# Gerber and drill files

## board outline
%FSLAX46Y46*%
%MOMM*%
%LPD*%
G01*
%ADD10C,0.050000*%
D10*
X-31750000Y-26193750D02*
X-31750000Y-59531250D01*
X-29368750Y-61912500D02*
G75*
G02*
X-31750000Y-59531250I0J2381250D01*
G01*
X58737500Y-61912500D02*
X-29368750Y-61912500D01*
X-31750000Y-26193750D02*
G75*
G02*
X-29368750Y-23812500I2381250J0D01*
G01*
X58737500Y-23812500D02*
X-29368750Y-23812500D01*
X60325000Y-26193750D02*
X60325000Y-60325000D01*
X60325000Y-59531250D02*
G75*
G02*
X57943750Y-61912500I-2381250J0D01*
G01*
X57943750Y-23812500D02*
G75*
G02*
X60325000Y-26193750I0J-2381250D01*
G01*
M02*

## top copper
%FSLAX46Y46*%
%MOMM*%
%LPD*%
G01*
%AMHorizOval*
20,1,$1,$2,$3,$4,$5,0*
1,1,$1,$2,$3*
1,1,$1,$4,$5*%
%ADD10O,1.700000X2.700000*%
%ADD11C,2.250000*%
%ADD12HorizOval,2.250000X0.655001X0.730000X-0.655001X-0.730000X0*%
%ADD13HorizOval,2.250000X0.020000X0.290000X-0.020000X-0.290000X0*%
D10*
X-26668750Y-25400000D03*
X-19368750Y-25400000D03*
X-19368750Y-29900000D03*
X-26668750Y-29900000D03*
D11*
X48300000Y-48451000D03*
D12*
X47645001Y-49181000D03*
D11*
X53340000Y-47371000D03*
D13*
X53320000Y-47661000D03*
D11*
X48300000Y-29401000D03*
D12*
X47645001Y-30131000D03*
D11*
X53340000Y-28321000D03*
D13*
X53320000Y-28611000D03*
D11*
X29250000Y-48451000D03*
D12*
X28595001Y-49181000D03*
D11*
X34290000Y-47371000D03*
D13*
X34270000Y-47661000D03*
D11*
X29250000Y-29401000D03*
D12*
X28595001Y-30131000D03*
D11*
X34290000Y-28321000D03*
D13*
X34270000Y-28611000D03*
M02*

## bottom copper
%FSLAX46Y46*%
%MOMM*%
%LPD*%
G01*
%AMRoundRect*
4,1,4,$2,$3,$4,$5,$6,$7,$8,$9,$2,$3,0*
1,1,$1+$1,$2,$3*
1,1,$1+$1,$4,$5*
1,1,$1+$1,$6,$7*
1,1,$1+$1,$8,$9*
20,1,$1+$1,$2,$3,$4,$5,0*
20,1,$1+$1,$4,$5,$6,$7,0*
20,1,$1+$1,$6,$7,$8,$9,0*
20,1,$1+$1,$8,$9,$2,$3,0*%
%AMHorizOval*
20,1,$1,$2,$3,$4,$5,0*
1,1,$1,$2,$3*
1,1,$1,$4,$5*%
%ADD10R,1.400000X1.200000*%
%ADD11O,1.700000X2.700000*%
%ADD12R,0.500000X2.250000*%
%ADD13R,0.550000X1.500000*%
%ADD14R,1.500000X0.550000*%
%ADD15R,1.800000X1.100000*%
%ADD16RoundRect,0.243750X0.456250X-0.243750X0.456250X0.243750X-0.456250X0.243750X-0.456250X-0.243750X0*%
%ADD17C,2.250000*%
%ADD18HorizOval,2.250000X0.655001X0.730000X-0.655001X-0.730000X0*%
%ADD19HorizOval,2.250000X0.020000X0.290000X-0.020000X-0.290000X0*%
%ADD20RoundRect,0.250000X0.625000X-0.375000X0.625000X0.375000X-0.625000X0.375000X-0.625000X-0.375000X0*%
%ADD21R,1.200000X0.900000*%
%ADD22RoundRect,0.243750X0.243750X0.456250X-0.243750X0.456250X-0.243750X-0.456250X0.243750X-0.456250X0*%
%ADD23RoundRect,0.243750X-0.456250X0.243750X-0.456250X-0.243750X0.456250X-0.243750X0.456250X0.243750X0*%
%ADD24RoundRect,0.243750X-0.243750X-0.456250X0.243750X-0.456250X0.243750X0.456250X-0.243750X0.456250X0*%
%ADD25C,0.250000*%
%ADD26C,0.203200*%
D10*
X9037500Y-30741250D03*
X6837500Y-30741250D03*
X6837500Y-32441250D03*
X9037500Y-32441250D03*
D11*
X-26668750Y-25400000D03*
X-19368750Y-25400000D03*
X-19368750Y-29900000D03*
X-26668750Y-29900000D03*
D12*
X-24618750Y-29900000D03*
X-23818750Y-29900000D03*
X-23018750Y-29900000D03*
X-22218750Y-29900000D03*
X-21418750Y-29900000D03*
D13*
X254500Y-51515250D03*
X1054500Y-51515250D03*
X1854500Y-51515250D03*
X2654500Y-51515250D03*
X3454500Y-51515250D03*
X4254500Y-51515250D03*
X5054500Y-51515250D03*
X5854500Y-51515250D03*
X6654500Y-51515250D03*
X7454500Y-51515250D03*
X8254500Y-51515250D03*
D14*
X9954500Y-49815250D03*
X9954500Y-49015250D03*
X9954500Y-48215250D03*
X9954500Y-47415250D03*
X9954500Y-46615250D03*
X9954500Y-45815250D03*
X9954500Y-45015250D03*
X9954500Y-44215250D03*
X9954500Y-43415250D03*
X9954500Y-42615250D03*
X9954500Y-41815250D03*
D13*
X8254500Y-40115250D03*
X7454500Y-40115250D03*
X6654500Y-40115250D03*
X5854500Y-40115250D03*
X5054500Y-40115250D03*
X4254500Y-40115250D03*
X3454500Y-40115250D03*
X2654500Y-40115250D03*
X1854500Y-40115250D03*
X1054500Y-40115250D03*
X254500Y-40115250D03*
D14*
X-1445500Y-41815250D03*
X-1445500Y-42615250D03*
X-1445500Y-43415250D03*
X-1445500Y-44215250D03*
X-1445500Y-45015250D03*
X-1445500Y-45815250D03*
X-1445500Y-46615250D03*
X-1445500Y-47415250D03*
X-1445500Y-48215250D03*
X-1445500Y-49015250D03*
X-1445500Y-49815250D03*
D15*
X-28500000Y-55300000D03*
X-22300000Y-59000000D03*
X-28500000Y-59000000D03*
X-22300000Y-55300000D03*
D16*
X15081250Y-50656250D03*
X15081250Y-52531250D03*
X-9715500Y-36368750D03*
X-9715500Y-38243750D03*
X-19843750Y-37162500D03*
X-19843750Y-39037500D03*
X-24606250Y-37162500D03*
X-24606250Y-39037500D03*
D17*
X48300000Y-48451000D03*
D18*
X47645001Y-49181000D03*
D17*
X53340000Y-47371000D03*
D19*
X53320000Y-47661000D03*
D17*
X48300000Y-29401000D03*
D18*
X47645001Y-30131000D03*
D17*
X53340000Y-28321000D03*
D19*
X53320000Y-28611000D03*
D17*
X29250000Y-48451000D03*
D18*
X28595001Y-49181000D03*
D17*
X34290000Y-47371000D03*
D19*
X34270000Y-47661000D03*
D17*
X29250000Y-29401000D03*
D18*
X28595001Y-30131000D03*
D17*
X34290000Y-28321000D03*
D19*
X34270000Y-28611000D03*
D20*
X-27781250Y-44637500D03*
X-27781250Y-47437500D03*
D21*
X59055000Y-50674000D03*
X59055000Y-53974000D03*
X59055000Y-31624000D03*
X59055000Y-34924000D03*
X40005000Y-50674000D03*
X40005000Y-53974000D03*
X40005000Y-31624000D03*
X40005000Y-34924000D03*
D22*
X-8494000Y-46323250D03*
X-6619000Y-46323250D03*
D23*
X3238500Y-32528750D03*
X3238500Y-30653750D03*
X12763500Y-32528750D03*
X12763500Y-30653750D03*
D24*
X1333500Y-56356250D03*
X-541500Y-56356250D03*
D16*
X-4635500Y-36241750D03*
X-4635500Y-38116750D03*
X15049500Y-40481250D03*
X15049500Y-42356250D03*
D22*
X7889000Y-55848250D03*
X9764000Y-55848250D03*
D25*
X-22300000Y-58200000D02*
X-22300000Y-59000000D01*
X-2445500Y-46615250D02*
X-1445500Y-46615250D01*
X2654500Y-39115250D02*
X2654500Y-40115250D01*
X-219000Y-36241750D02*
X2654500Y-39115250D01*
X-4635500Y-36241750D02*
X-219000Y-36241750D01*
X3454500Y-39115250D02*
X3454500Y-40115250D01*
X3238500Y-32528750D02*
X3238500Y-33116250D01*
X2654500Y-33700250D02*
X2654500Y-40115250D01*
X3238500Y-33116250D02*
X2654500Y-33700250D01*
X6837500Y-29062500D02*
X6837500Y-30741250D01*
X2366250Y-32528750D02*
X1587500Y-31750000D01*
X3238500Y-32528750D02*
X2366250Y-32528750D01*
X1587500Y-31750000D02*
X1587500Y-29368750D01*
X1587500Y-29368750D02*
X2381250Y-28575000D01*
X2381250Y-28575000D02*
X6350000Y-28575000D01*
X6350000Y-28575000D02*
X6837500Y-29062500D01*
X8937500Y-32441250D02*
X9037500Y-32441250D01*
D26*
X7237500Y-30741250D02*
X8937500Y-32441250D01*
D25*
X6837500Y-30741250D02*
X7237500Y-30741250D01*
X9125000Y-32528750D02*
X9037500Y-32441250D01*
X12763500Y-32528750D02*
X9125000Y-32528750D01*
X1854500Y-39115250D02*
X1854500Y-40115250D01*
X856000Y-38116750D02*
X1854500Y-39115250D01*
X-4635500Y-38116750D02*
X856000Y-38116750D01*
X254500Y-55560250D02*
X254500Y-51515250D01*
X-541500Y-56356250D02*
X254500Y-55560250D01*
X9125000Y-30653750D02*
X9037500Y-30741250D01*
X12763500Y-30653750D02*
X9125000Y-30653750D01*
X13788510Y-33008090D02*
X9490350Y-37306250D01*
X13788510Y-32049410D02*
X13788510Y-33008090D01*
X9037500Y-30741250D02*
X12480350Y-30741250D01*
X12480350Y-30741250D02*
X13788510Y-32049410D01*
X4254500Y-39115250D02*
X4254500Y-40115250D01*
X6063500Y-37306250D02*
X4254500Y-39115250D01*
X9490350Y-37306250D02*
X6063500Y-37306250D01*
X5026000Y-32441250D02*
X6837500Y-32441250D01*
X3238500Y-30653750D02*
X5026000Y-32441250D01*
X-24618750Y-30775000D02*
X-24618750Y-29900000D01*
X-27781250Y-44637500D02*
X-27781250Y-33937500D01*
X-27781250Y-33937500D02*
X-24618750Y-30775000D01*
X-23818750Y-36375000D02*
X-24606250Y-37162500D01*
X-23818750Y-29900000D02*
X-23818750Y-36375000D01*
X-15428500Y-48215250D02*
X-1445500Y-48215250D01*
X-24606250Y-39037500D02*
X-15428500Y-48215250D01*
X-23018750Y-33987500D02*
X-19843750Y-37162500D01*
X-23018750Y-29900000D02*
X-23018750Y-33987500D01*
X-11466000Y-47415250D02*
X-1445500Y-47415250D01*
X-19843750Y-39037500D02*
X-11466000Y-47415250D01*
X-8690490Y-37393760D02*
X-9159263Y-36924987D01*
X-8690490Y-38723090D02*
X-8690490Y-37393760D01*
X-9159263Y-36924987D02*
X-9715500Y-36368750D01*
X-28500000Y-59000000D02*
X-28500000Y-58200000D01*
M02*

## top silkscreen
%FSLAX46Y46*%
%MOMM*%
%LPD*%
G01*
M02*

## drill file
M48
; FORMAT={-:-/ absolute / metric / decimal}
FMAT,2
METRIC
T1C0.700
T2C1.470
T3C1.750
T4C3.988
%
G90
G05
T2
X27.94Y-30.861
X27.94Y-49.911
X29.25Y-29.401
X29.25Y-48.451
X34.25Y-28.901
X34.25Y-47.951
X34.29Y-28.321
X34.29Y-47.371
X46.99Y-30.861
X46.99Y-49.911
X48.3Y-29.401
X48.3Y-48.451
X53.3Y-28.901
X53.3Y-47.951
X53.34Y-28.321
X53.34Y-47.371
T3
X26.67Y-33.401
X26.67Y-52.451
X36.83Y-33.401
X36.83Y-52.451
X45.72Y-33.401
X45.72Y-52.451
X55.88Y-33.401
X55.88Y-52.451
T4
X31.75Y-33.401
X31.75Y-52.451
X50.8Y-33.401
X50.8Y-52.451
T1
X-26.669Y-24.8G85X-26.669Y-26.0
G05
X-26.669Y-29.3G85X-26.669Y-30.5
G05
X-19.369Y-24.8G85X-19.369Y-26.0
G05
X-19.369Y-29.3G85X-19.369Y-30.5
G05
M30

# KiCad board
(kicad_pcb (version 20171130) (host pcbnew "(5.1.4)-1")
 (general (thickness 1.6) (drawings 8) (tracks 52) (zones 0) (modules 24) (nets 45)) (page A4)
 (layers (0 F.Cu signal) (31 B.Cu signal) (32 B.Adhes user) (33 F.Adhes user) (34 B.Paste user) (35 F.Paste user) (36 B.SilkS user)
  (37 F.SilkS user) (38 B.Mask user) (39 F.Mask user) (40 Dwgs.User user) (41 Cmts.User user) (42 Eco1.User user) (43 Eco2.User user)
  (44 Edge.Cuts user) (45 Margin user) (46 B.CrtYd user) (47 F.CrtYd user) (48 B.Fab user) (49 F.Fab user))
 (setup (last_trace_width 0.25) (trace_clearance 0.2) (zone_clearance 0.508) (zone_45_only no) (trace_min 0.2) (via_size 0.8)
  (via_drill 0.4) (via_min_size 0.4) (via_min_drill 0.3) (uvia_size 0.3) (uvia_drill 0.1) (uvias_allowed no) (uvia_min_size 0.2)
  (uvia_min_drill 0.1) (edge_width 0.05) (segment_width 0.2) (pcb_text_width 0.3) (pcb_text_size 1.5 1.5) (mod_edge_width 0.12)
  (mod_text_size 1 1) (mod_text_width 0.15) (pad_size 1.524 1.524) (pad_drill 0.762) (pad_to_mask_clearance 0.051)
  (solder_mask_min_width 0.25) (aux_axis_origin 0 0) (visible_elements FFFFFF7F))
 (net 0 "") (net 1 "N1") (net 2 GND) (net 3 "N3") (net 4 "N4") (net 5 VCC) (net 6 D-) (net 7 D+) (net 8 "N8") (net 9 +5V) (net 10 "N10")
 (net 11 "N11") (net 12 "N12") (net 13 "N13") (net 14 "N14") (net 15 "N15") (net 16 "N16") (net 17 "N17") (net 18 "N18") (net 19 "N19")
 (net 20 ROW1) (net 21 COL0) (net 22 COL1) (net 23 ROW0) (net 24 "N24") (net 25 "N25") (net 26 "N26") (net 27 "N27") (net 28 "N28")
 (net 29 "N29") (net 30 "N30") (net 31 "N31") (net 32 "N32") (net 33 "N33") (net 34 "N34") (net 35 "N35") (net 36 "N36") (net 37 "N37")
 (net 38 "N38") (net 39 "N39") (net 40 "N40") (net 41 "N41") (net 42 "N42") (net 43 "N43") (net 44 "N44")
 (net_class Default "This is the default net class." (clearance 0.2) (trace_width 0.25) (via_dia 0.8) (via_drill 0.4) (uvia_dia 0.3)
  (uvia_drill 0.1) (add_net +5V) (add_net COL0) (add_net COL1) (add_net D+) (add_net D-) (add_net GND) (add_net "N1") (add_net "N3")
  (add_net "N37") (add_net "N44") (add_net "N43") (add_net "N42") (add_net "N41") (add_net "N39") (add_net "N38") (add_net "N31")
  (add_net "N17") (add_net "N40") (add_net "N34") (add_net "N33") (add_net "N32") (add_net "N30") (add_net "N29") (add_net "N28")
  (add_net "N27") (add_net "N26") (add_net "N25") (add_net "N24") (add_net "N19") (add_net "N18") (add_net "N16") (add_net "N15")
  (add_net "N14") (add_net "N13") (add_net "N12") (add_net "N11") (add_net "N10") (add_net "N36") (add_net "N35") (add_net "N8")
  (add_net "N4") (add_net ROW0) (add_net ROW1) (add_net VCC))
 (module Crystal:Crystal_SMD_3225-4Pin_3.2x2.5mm (layer B.Cu) (at 7.9375 31.59125 180)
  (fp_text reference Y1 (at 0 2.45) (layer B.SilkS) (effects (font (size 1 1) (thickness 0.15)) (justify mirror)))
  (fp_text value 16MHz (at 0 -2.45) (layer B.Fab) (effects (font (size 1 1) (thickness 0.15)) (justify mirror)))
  (pad 4 smd rect (at -1.1 0.85 180) (size 1.4 1.2) (layers B.Cu B.Paste B.Mask) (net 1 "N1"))
  (pad 3 smd rect (at 1.1 0.85 180) (size 1.4 1.2) (layers B.Cu B.Paste B.Mask) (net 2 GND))
  (pad 2 smd rect (at 1.1 -0.85 180) (size 1.4 1.2) (layers B.Cu B.Paste B.Mask) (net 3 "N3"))
  (pad 1 smd rect (at -1.1 -0.85 180) (size 1.4 1.2) (layers B.Cu B.Paste B.Mask) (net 2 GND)))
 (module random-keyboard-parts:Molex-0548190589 (layer B.Cu) (at -23.01875 25.4 270)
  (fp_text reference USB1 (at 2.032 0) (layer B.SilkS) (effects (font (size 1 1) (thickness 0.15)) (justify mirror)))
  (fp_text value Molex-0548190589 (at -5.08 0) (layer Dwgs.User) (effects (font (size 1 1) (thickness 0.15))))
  (pad 6 thru_hole oval (at 0 3.65 270) (size 2.7 1.7) (drill oval 1.9 0.7) (layers *.Cu *.Mask) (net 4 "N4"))
  (pad 6 thru_hole oval (at 0 -3.65 270) (size 2.7 1.7) (drill oval 1.9 0.7) (layers *.Cu *.Mask) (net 4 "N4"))
  (pad 6 thru_hole oval (at 4.5 -3.65 270) (size 2.7 1.7) (drill oval 1.9 0.7) (layers *.Cu *.Mask) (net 4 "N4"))
  (pad 6 thru_hole oval (at 4.5 3.65 270) (size 2.7 1.7) (drill oval 1.9 0.7) (layers *.Cu *.Mask) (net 4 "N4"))
  (pad 5 smd rect (at 4.5 1.6 270) (size 2.25 0.5) (layers B.Cu B.Paste B.Mask) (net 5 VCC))
  (pad 4 smd rect (at 4.5 0.8 270) (size 2.25 0.5) (layers B.Cu B.Paste B.Mask) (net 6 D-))
  (pad 3 smd rect (at 4.5 0 270) (size 2.25 0.5) (layers B.Cu B.Paste B.Mask) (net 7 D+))
  (pad 2 smd rect (at 4.5 -0.8 270) (size 2.25 0.5) (layers B.Cu B.Paste B.Mask) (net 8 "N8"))
  (pad 1 smd rect (at 4.5 -1.6 270) (size 2.25 0.5) (layers B.Cu B.Paste B.Mask) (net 2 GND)))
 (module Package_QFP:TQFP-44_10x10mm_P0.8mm (layer B.Cu) (at 4.2545 45.81525)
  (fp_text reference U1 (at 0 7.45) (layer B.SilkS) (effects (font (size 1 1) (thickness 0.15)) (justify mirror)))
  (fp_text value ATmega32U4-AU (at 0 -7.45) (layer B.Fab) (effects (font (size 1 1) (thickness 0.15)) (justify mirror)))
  (pad 44 smd rect (at -4 5.7 270) (size 1.5 0.55) (layers B.Cu B.Paste B.Mask) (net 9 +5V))
  (pad 43 smd rect (at -3.2 5.7 270) (size 1.5 0.55) (layers B.Cu B.Paste B.Mask) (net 2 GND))
  (pad 42 smd rect (at -2.4 5.7 270) (size 1.5 0.55) (layers B.Cu B.Paste B.Mask) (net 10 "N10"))
  (pad 41 smd rect (at -1.6 5.7 270) (size 1.5 0.55) (layers B.Cu B.Paste B.Mask) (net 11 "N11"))
  (pad 40 smd rect (at -0.8 5.7 270) (size 1.5 0.55) (layers B.Cu B.Paste B.Mask) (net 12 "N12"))
  (pad 39 smd rect (at 0 5.7 270) (size 1.5 0.55) (layers B.Cu B.Paste B.Mask) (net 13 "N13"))
  (pad 38 smd rect (at 0.8 5.7 270) (size 1.5 0.55) (layers B.Cu B.Paste B.Mask) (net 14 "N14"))
  (pad 37 smd rect (at 1.6 5.7 270) (size 1.5 0.55) (layers B.Cu B.Paste B.Mask) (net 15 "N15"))
  (pad 36 smd rect (at 2.4 5.7 270) (size 1.5 0.55) (layers B.Cu B.Paste B.Mask) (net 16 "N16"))
  (pad 35 smd rect (at 3.2 5.7 270) (size 1.5 0.55) (layers B.Cu B.Paste B.Mask) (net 2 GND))
  (pad 34 smd rect (at 4 5.7 270) (size 1.5 0.55) (layers B.Cu B.Paste B.Mask) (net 9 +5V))
  (pad 33 smd rect (at 5.7 4) (size 1.5 0.55) (layers B.Cu B.Paste B.Mask) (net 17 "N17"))
  (pad 32 smd rect (at 5.7 3.2) (size 1.5 0.55) (layers B.Cu B.Paste B.Mask) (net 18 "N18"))
  (pad 31 smd rect (at 5.7 2.4) (size 1.5 0.55) (layers B.Cu B.Paste B.Mask) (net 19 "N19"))
  (pad 30 smd rect (at 5.7 1.6) (size 1.5 0.55) (layers B.Cu B.Paste B.Mask) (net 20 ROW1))
  (pad 29 smd rect (at 5.7 0.8) (size 1.5 0.55) (layers B.Cu B.Paste B.Mask) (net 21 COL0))
  (pad 28 smd rect (at 5.7 0) (size 1.5 0.55) (layers B.Cu B.Paste B.Mask) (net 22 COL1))
  (pad 27 smd rect (at 5.7 -0.8) (size 1.5 0.55) (layers B.Cu B.Paste B.Mask) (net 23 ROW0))
  (pad 26 smd rect (at 5.7 -1.6) (size 1.5 0.55) (layers B.Cu B.Paste B.Mask) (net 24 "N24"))
  (pad 25 smd rect (at 5.7 -2.4) (size 1.5 0.55) (layers B.Cu B.Paste B.Mask) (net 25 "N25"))
  (pad 24 smd rect (at 5.7 -3.2) (size 1.5 0.55) (layers B.Cu B.Paste B.Mask) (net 9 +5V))
  (pad 23 smd rect (at 5.7 -4) (size 1.5 0.55) (layers B.Cu B.Paste B.Mask) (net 2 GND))
  (pad 22 smd rect (at 4 -5.7 270) (size 1.5 0.55) (layers B.Cu B.Paste B.Mask) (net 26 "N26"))
  (pad 21 smd rect (at 3.2 -5.7 270) (size 1.5 0.55) (layers B.Cu B.Paste B.Mask) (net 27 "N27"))
  (pad 20 smd rect (at 2.4 -5.7 270) (size 1.5 0.55) (layers B.Cu B.Paste B.Mask) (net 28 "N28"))
  (pad 19 smd rect (at 1.6 -5.7 270) (size 1.5 0.55) (layers B.Cu B.Paste B.Mask) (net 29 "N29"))
  (pad 18 smd rect (at 0.8 -5.7 270) (size 1.5 0.55) (layers B.Cu B.Paste B.Mask) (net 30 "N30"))
  (pad 17 smd rect (at 0 -5.7 270) (size 1.5 0.55) (layers B.Cu B.Paste B.Mask) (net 1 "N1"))
  (pad 16 smd rect (at -0.8 -5.7 270) (size 1.5 0.55) (layers B.Cu B.Paste B.Mask) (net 3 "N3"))
  (pad 15 smd rect (at -1.6 -5.7 270) (size 1.5 0.55) (layers B.Cu B.Paste B.Mask) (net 2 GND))
  (pad 14 smd rect (at -2.4 -5.7 270) (size 1.5 0.55) (layers B.Cu B.Paste B.Mask) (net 9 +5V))
  (pad 13 smd rect (at -3.2 -5.7 270) (size 1.5 0.55) (layers B.Cu B.Paste B.Mask) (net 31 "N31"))
  (pad 12 smd rect (at -4 -5.7 270) (size 1.5 0.55) (layers B.Cu B.Paste B.Mask) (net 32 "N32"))
  (pad 11 smd rect (at -5.7 -4) (size 1.5 0.55) (layers B.Cu B.Paste B.Mask) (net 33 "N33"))
  (pad 10 smd rect (at -5.7 -3.2) (size 1.5 0.55) (layers B.Cu B.Paste B.Mask) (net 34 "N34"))
  (pad 9 smd rect (at -5.7 -2.4) (size 1.5 0.55) (layers B.Cu B.Paste B.Mask) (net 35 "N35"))
  (pad 8 smd rect (at -5.7 -1.6) (size 1.5 0.55) (layers B.Cu B.Paste B.Mask) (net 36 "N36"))
  (pad 7 smd rect (at -5.7 -0.8) (size 1.5 0.55) (layers B.Cu B.Paste B.Mask) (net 9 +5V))
  (pad 6 smd rect (at -5.7 0) (size 1.5 0.55) (layers B.Cu B.Paste B.Mask) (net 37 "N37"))
  (pad 5 smd rect (at -5.7 0.8) (size 1.5 0.55) (layers B.Cu B.Paste B.Mask) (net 2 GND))
  (pad 4 smd rect (at -5.7 1.6) (size 1.5 0.55) (layers B.Cu B.Paste B.Mask) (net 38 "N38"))
  (pad 3 smd rect (at -5.7 2.4) (size 1.5 0.55) (layers B.Cu B.Paste B.Mask) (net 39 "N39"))
  (pad 2 smd rect (at -5.7 3.2) (size 1.5 0.55) (layers B.Cu B.Paste B.Mask) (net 9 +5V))
  (pad 1 smd rect (at -5.7 4) (size 1.5 0.55) (layers B.Cu B.Paste B.Mask) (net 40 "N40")))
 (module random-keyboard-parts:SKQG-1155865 (layer B.Cu) (at -25.4 57.15)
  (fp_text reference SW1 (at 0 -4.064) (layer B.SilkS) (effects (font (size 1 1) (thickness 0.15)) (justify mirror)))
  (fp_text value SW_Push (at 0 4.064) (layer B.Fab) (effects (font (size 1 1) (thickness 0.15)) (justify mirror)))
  (pad 4 smd rect (at -3.1 -1.85) (size 1.8 1.1) (layers B.Cu B.Paste B.Mask))
  (pad 3 smd rect (at 3.1 1.85) (size 1.8 1.1) (layers B.Cu B.Paste B.Mask))
  (pad 2 smd rect (at -3.1 1.85) (size 1.8 1.1) (layers B.Cu B.Paste B.Mask) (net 31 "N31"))
  (pad 1 smd rect (at 3.1 -1.85) (size 1.8 1.1) (layers B.Cu B.Paste B.Mask) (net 2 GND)))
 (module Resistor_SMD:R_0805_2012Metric (layer B.Cu) (at 15.08125 51.59375 90)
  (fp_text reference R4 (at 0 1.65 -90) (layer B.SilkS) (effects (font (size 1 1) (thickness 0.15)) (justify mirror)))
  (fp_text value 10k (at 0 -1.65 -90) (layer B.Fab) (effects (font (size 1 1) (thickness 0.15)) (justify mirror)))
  (pad 2 smd roundrect (at 0.9375 0 90) (size 0.975 1.4) (layers B.Cu B.Paste B.Mask) (roundrect_rratio 0.25) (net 17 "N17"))
  (pad 1 smd roundrect (at -0.9375 0 90) (size 0.975 1.4) (layers B.Cu B.Paste B.Mask) (roundrect_rratio 0.25) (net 2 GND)))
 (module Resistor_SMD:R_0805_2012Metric (layer B.Cu) (at -9.7155 37.30625 90)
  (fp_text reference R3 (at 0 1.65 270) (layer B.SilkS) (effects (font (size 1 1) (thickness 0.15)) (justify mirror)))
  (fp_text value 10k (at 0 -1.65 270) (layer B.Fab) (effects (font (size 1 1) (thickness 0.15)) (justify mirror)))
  (pad 2 smd roundrect (at 0.9375 0 90) (size 0.975 1.4) (layers B.Cu B.Paste B.Mask) (roundrect_rratio 0.25) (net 31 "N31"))
  (pad 1 smd roundrect (at -0.9375 0 90) (size 0.975 1.4) (layers B.Cu B.Paste B.Mask) (roundrect_rratio 0.25) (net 9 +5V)))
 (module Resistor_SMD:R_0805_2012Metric (layer B.Cu) (at -19.84375 38.1 90)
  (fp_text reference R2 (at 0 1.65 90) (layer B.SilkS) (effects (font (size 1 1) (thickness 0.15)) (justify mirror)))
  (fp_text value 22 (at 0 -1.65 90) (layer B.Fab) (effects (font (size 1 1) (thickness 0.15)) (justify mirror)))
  (pad 2 smd roundrect (at 0.9375 0 90) (size 0.975 1.4) (layers B.Cu B.Paste B.Mask) (roundrect_rratio 0.25) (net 7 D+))
  (pad 1 smd roundrect (at -0.9375 0 90) (size 0.975 1.4) (layers B.Cu B.Paste B.Mask) (roundrect_rratio 0.25) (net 38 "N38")))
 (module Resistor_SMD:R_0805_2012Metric (layer B.Cu) (at -24.60625 38.1 90)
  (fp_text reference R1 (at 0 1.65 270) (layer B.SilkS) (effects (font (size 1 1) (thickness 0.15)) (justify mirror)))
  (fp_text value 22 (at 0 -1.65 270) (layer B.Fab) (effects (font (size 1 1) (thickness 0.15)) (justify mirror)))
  (pad 2 smd roundrect (at 0.9375 0 90) (size 0.975 1.4) (layers B.Cu B.Paste B.Mask) (roundrect_rratio 0.25) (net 6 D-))
  (pad 1 smd roundrect (at -0.9375 0 90) (size 0.975 1.4) (layers B.Cu B.Paste B.Mask) (roundrect_rratio 0.25) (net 39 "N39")))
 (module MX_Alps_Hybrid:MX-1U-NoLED (layer F.Cu) (at 50.8 52.451)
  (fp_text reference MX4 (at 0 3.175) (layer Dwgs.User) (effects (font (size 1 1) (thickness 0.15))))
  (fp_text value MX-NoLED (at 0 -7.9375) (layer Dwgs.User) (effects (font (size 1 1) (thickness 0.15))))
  (pad "" np_thru_hole circle (at 5.08 0 48.0996) (size 1.75 1.75) (drill 1.75) (layers *.Cu *.Mask))
  (pad "" np_thru_hole circle (at -5.08 0 48.0996) (size 1.75 1.75) (drill 1.75) (layers *.Cu *.Mask))
  (pad 1 thru_hole circle (at -2.5 -4) (size 2.25 2.25) (drill 1.47) (layers *.Cu B.Mask) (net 22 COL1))
  (pad "" np_thru_hole circle (at 0 0) (size 3.9878 3.9878) (drill 3.9878) (layers *.Cu *.Mask))
  (pad 1 thru_hole oval (at -3.81 -2.54 48.0996) (size 4.211556 2.25) (drill 1.47 (offset 0.980778 0)) (layers *.Cu B.Mask) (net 22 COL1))
  (pad 2 thru_hole circle (at 2.54 -5.08) (size 2.25 2.25) (drill 1.47) (layers *.Cu B.Mask) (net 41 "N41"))
  (pad 2 thru_hole oval (at 2.5 -4.5 86.0548) (size 2.831378 2.25) (drill 1.47 (offset 0.290689 0)) (layers *.Cu B.Mask) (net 41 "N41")))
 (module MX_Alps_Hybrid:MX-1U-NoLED (layer F.Cu) (at 50.8 33.401)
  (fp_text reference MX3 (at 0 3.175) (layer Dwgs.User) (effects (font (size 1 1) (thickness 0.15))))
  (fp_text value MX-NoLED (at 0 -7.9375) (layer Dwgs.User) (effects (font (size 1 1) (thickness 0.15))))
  (pad "" np_thru_hole circle (at 5.08 0 48.0996) (size 1.75 1.75) (drill 1.75) (layers *.Cu *.Mask))
  (pad "" np_thru_hole circle (at -5.08 0 48.0996) (size 1.75 1.75) (drill 1.75) (layers *.Cu *.Mask))
  (pad 1 thru_hole circle (at -2.5 -4) (size 2.25 2.25) (drill 1.47) (layers *.Cu B.Mask) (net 22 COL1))
  (pad "" np_thru_hole circle (at 0 0) (size 3.9878 3.9878) (drill 3.9878) (layers *.Cu *.Mask))
  (pad 1 thru_hole oval (at -3.81 -2.54 48.0996) (size 4.211556 2.25) (drill 1.47 (offset 0.980778 0)) (layers *.Cu B.Mask) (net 22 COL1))
  (pad 2 thru_hole circle (at 2.54 -5.08) (size 2.25 2.25) (drill 1.47) (layers *.Cu B.Mask) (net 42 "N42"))
  (pad 2 thru_hole oval (at 2.5 -4.5 86.0548) (size 2.831378 2.25) (drill 1.47 (offset 0.290689 0)) (layers *.Cu B.Mask) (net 42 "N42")))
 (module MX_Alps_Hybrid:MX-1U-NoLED (layer F.Cu) (at 31.75 52.451)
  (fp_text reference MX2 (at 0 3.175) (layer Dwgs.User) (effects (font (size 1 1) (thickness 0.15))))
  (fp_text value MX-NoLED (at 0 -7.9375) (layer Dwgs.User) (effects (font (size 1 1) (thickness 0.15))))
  (pad "" np_thru_hole circle (at 5.08 0 48.0996) (size 1.75 1.75) (drill 1.75) (layers *.Cu *.Mask))
  (pad "" np_thru_hole circle (at -5.08 0 48.0996) (size 1.75 1.75) (drill 1.75) (layers *.Cu *.Mask))
  (pad 1 thru_hole circle (at -2.5 -4) (size 2.25 2.25) (drill 1.47) (layers *.Cu B.Mask) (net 21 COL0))
  (pad "" np_thru_hole circle (at 0 0) (size 3.9878 3.9878) (drill 3.9878) (layers *.Cu *.Mask))
  (pad 1 thru_hole oval (at -3.81 -2.54 48.0996) (size 4.211556 2.25) (drill 1.47 (offset 0.980778 0)) (layers *.Cu B.Mask) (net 21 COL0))
  (pad 2 thru_hole circle (at 2.54 -5.08) (size 2.25 2.25) (drill 1.47) (layers *.Cu B.Mask) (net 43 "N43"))
  (pad 2 thru_hole oval (at 2.5 -4.5 86.0548) (size 2.831378 2.25) (drill 1.47 (offset 0.290689 0)) (layers *.Cu B.Mask) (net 43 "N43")))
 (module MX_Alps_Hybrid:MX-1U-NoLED (layer F.Cu) (at 31.75 33.401)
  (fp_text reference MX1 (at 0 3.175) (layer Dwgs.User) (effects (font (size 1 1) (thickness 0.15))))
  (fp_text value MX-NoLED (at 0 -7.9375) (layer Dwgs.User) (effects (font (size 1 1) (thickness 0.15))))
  (pad "" np_thru_hole circle (at 5.08 0 48.0996) (size 1.75 1.75) (drill 1.75) (layers *.Cu *.Mask))
  (pad "" np_thru_hole circle (at -5.08 0 48.0996) (size 1.75 1.75) (drill 1.75) (layers *.Cu *.Mask))
  (pad 1 thru_hole circle (at -2.5 -4) (size 2.25 2.25) (drill 1.47) (layers *.Cu B.Mask) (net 21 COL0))
  (pad "" np_thru_hole circle (at 0 0) (size 3.9878 3.9878) (drill 3.9878) (layers *.Cu *.Mask))
  (pad 1 thru_hole oval (at -3.81 -2.54 48.0996) (size 4.211556 2.25) (drill 1.47 (offset 0.980778 0)) (layers *.Cu B.Mask) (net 21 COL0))
  (pad 2 thru_hole circle (at 2.54 -5.08) (size 2.25 2.25) (drill 1.47) (layers *.Cu B.Mask) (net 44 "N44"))
  (pad 2 thru_hole oval (at 2.5 -4.5 86.0548) (size 2.831378 2.25) (drill 1.47 (offset 0.290689 0)) (layers *.Cu B.Mask) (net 44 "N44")))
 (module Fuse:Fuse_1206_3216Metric (layer B.Cu) (at -27.78125 46.0375 90)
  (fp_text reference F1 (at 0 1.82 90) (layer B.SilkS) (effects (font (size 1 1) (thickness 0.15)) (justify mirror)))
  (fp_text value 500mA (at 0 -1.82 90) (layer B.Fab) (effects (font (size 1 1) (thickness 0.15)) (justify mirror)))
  (pad 2 smd roundrect (at 1.4 0 90) (size 1.25 1.75) (layers B.Cu B.Paste B.Mask) (roundrect_rratio 0.2) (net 5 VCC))
  (pad 1 smd roundrect (at -1.4 0 90) (size 1.25 1.75) (layers B.Cu B.Paste B.Mask) (roundrect_rratio 0.2) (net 9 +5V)))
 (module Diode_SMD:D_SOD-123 (layer B.Cu) (at 59.055 52.324 90)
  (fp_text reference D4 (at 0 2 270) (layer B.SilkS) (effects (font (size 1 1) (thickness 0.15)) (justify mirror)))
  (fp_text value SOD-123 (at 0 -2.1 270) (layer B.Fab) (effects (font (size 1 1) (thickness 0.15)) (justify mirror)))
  (pad 2 smd rect (at 1.65 0 90) (size 0.9 1.2) (layers B.Cu B.Paste B.Mask) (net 41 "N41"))
  (pad 1 smd rect (at -1.65 0 90) (size 0.9 1.2) (layers B.Cu B.Paste B.Mask) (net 20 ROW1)))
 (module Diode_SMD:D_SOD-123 (layer B.Cu) (at 59.055 33.274 90)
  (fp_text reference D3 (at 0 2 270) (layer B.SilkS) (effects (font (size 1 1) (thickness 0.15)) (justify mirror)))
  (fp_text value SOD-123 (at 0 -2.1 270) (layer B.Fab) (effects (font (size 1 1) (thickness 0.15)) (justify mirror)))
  (pad 2 smd rect (at 1.65 0 90) (size 0.9 1.2) (layers B.Cu B.Paste B.Mask) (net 42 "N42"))
  (pad 1 smd rect (at -1.65 0 90) (size 0.9 1.2) (layers B.Cu B.Paste B.Mask) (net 23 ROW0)))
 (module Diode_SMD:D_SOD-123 (layer B.Cu) (at 40.005 52.324 90)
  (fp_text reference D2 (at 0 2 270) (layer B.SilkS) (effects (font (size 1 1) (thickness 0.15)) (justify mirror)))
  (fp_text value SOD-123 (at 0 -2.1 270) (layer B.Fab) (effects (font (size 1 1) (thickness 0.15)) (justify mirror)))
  (pad 2 smd rect (at 1.65 0 90) (size 0.9 1.2) (layers B.Cu B.Paste B.Mask) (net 43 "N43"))
  (pad 1 smd rect (at -1.65 0 90) (size 0.9 1.2) (layers B.Cu B.Paste B.Mask) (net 20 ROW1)))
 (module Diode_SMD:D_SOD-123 (layer B.Cu) (at 40.005 33.274 90)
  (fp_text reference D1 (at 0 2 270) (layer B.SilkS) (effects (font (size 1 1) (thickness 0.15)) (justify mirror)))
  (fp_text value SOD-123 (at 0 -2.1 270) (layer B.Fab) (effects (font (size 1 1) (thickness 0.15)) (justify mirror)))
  (pad 2 smd rect (at 1.65 0 90) (size 0.9 1.2) (layers B.Cu B.Paste B.Mask) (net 44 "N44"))
  (pad 1 smd rect (at -1.65 0 90) (size 0.9 1.2) (layers B.Cu B.Paste B.Mask) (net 23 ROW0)))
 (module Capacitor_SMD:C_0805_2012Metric (layer B.Cu) (at -7.5565 46.32325 180)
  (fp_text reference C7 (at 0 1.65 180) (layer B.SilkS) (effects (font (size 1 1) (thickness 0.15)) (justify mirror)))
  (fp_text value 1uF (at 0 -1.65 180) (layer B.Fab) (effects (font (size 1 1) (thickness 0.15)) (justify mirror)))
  (pad 2 smd roundrect (at 0.9375 0 180) (size 0.975 1.4) (layers B.Cu B.Paste B.Mask) (roundrect_rratio 0.25) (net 2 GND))
  (pad 1 smd roundrect (at -0.9375 0 180) (size 0.975 1.4) (layers B.Cu B.Paste B.Mask) (roundrect_rratio 0.25) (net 37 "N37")))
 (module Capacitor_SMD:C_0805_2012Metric (layer B.Cu) (at 3.2385 31.59125 270)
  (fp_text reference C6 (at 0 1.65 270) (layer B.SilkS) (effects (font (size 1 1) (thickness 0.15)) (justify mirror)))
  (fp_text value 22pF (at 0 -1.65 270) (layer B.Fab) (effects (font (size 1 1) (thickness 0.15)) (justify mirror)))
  (pad 2 smd roundrect (at 0.9375 0 270) (size 0.975 1.4) (layers B.Cu B.Paste B.Mask) (roundrect_rratio 0.25) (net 2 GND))
  (pad 1 smd roundrect (at -0.9375 0 270) (size 0.975 1.4) (layers B.Cu B.Paste B.Mask) (roundrect_rratio 0.25) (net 3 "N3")))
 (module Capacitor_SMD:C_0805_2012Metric (layer B.Cu) (at 12.7635 31.59125 270)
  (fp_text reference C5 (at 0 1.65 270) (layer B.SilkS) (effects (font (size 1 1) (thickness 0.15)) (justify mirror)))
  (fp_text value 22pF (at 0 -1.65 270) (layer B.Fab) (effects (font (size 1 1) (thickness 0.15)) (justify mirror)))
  (pad 2 smd roundrect (at 0.9375 0 270) (size 0.975 1.4) (layers B.Cu B.Paste B.Mask) (roundrect_rratio 0.25) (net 2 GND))
  (pad 1 smd roundrect (at -0.9375 0 270) (size 0.975 1.4) (layers B.Cu B.Paste B.Mask) (roundrect_rratio 0.25) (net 1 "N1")))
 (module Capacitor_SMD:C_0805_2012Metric (layer B.Cu) (at 0.396 56.35625)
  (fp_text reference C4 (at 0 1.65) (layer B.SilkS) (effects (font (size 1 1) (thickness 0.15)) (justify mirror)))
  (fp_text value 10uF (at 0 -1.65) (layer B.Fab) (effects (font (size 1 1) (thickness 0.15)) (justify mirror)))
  (pad 2 smd roundrect (at 0.9375 0) (size 0.975 1.4) (layers B.Cu B.Paste B.Mask) (roundrect_rratio 0.25) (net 2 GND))
  (pad 1 smd roundrect (at -0.9375 0) (size 0.975 1.4) (layers B.Cu B.Paste B.Mask) (roundrect_rratio 0.25) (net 9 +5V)))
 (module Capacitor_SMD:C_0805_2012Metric (layer B.Cu) (at -4.6355 37.17925 90)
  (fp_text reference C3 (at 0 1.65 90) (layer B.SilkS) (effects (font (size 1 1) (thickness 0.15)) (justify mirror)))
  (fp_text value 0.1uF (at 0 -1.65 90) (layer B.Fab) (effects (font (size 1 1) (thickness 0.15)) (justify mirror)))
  (pad 2 smd roundrect (at 0.9375 0 90) (size 0.975 1.4) (layers B.Cu B.Paste B.Mask) (roundrect_rratio 0.25) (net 2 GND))
  (pad 1 smd roundrect (at -0.9375 0 90) (size 0.975 1.4) (layers B.Cu B.Paste B.Mask) (roundrect_rratio 0.25) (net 9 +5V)))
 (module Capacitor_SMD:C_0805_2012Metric (layer B.Cu) (at 15.0495 41.41875 90)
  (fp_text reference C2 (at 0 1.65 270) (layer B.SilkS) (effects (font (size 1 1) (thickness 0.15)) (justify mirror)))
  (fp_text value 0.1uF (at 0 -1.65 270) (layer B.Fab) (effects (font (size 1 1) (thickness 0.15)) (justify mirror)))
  (pad 2 smd roundrect (at 0.9375 0 90) (size 0.975 1.4) (layers B.Cu B.Paste B.Mask) (roundrect_rratio 0.25) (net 2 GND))
  (pad 1 smd roundrect (at -0.9375 0 90) (size 0.975 1.4) (layers B.Cu B.Paste B.Mask) (roundrect_rratio 0.25) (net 9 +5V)))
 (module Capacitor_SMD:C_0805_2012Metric (layer B.Cu) (at 8.8265 55.84825 180)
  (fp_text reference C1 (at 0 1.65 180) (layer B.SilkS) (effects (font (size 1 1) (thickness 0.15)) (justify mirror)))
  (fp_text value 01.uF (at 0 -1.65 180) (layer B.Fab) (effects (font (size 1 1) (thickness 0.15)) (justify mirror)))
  (pad 2 smd roundrect (at 0.9375 0 180) (size 0.975 1.4) (layers B.Cu B.Paste B.Mask) (roundrect_rratio 0.25) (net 2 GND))
  (pad 1 smd roundrect (at -0.9375 0 180) (size 0.975 1.4) (layers B.Cu B.Paste B.Mask) (roundrect_rratio 0.25) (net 9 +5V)))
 (gr_line (start -31.75 26.19375) (end -31.75 59.53125) (layer Edge.Cuts) (width 0.05))
 (gr_arc (start -29.36875 59.53125) (end -31.75 59.53125) (angle -90) (layer Edge.Cuts) (width 0.05))
 (gr_line (start 58.7375 61.9125) (end -29.36875 61.9125) (layer Edge.Cuts) (width 0.05))
 (gr_arc (start -29.36875 26.19375) (end -29.36875 23.8125) (angle -90) (layer Edge.Cuts) (width 0.05))
 (gr_line (start 58.7375 23.8125) (end -29.36875 23.8125) (layer Edge.Cuts) (width 0.05))
 (gr_line (start 60.325 26.19375) (end 60.325 60.325) (layer Edge.Cuts) (width 0.05))
 (gr_arc (start 57.94375 59.53125) (end 57.94375 61.9125) (angle -90) (layer Edge.Cuts) (width 0.05))
 (gr_arc (start 57.94375 26.19375) (end 60.325 26.19375) (angle -90) (layer Edge.Cuts) (width 0.05))
 (segment (start -22.3 58.2) (end -22.3 59) (width 0.25) (layer B.Cu) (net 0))
 (segment (start -2.4455 46.61525) (end -1.4455 46.61525) (width 0.25) (layer B.Cu) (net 2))
 (segment (start 2.6545 39.11525) (end 2.6545 40.11525) (width 0.25) (layer B.Cu) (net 2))
 (segment (start -0.219 36.24175) (end 2.6545 39.11525) (width 0.25) (layer B.Cu) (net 2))
 (segment (start -4.6355 36.24175) (end -0.219 36.24175) (width 0.25) (layer B.Cu) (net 2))
 (segment (start 3.4545 39.11525) (end 3.4545 40.11525) (width 0.25) (layer B.Cu) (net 3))
 (segment (start 3.2385 32.52875) (end 3.2385 33.11625) (width 0.25) (layer B.Cu) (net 2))
 (segment (start 2.6545 33.70025) (end 2.6545 40.11525) (width 0.25) (layer B.Cu) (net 2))
 (segment (start 3.2385 33.11625) (end 2.6545 33.70025) (width 0.25) (layer B.Cu) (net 2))
 (segment (start 6.8375 29.0625) (end 6.8375 30.74125) (width 0.25) (layer B.Cu) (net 2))
 (segment (start 2.36625 32.52875) (end 1.5875 31.75) (width 0.25) (layer B.Cu) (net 2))
 (segment (start 3.2385 32.52875) (end 2.36625 32.52875) (width 0.25) (layer B.Cu) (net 2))
 (segment (start 1.5875 31.75) (end 1.5875 29.36875) (width 0.25) (layer B.Cu) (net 2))
 (segment (start 1.5875 29.36875) (end 2.38125 28.575) (width 0.25) (layer B.Cu) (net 2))
 (segment (start 2.38125 28.575) (end 6.35 28.575) (width 0.25) (layer B.Cu) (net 2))
 (segment (start 6.35 28.575) (end 6.8375 29.0625) (width 0.25) (layer B.Cu) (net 2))
 (segment (start 8.9375 32.44125) (end 9.0375 32.44125) (width 0.25) (layer B.Cu) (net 2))
 (segment (start 7.2375 30.74125) (end 8.9375 32.44125) (width 0.2032) (layer B.Cu) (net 2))
 (segment (start 6.8375 30.74125) (end 7.2375 30.74125) (width 0.25) (layer B.Cu) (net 2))
 (segment (start 9.125 32.52875) (end 9.0375 32.44125) (width 0.25) (layer B.Cu) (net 2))
 (segment (start 12.7635 32.52875) (end 9.125 32.52875) (width 0.25) (layer B.Cu) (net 2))
 (segment (start 1.8545 39.11525) (end 1.8545 40.11525) (width 0.25) (layer B.Cu) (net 9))
 (segment (start 0.856 38.11675) (end 1.8545 39.11525) (width 0.25) (layer B.Cu) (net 9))
 (segment (start -4.6355 38.11675) (end 0.856 38.11675) (width 0.25) (layer B.Cu) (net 9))
 (segment (start 0.2545 55.56025) (end 0.2545 51.51525) (width 0.25) (layer B.Cu) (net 9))
 (segment (start -0.5415 56.35625) (end 0.2545 55.56025) (width 0.25) (layer B.Cu) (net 9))
 (segment (start 9.125 30.65375) (end 9.0375 30.74125) (width 0.25) (layer B.Cu) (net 1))
 (segment (start 12.7635 30.65375) (end 9.125 30.65375) (width 0.25) (layer B.Cu) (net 1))
 (segment (start 13.78851 33.00809) (end 9.49035 37.30625) (width 0.25) (layer B.Cu) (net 1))
 (segment (start 13.78851 32.04941) (end 13.78851 33.00809) (width 0.25) (layer B.Cu) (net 1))
 (segment (start 9.0375 30.74125) (end 12.48035 30.74125) (width 0.25) (layer B.Cu) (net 1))
 (segment (start 12.48035 30.74125) (end 13.78851 32.04941) (width 0.25) (layer B.Cu) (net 1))
 (segment (start 4.2545 39.11525) (end 4.2545 40.11525) (width 0.25) (layer B.Cu) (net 1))
 (segment (start 6.0635 37.30625) (end 4.2545 39.11525) (width 0.25) (layer B.Cu) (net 1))
 (segment (start 9.49035 37.30625) (end 6.0635 37.30625) (width 0.25) (layer B.Cu) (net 1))
 (segment (start 5.026 32.44125) (end 6.8375 32.44125) (width 0.25) (layer B.Cu) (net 3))
 (segment (start 3.2385 30.65375) (end 5.026 32.44125) (width 0.25) (layer B.Cu) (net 3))
 (segment (start -24.61875 30.775) (end -24.61875 29.9) (width 0.25) (layer B.Cu) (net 5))
 (segment (start -27.78125 44.6375) (end -27.78125 33.9375) (width 0.25) (layer B.Cu) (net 5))
 (segment (start -27.78125 33.9375) (end -24.61875 30.775) (width 0.25) (layer B.Cu) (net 5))
 (segment (start -23.81875 36.375) (end -24.60625 37.1625) (width 0.25) (layer B.Cu) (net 6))
 (segment (start -23.81875 29.9) (end -23.81875 36.375) (width 0.25) (layer B.Cu) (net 6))
 (segment (start -15.4285 48.21525) (end -1.4455 48.21525) (width 0.25) (layer B.Cu) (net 39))
 (segment (start -24.60625 39.0375) (end -15.4285 48.21525) (width 0.25) (layer B.Cu) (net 39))
 (segment (start -23.01875 33.9875) (end -19.84375 37.1625) (width 0.25) (layer B.Cu) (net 7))
 (segment (start -23.01875 29.9) (end -23.01875 33.9875) (width 0.25) (layer B.Cu) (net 7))
 (segment (start -11.466 47.41525) (end -1.4455 47.41525) (width 0.25) (layer B.Cu) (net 38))
 (segment (start -19.84375 39.0375) (end -11.466 47.41525) (width 0.25) (layer B.Cu) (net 38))
 (segment (start -8.69049 37.39376) (end -9.159263 36.924987) (width 0.25) (layer B.Cu) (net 31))
 (segment (start -8.69049 38.72309) (end -8.69049 37.39376) (width 0.25) (layer B.Cu) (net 31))
 (segment (start -9.159263 36.924987) (end -9.7155 36.36875) (width 0.25) (layer B.Cu) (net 31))
 (segment (start -28.5 59) (end -28.5 58.2) (width 0.25) (layer B.Cu) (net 31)))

